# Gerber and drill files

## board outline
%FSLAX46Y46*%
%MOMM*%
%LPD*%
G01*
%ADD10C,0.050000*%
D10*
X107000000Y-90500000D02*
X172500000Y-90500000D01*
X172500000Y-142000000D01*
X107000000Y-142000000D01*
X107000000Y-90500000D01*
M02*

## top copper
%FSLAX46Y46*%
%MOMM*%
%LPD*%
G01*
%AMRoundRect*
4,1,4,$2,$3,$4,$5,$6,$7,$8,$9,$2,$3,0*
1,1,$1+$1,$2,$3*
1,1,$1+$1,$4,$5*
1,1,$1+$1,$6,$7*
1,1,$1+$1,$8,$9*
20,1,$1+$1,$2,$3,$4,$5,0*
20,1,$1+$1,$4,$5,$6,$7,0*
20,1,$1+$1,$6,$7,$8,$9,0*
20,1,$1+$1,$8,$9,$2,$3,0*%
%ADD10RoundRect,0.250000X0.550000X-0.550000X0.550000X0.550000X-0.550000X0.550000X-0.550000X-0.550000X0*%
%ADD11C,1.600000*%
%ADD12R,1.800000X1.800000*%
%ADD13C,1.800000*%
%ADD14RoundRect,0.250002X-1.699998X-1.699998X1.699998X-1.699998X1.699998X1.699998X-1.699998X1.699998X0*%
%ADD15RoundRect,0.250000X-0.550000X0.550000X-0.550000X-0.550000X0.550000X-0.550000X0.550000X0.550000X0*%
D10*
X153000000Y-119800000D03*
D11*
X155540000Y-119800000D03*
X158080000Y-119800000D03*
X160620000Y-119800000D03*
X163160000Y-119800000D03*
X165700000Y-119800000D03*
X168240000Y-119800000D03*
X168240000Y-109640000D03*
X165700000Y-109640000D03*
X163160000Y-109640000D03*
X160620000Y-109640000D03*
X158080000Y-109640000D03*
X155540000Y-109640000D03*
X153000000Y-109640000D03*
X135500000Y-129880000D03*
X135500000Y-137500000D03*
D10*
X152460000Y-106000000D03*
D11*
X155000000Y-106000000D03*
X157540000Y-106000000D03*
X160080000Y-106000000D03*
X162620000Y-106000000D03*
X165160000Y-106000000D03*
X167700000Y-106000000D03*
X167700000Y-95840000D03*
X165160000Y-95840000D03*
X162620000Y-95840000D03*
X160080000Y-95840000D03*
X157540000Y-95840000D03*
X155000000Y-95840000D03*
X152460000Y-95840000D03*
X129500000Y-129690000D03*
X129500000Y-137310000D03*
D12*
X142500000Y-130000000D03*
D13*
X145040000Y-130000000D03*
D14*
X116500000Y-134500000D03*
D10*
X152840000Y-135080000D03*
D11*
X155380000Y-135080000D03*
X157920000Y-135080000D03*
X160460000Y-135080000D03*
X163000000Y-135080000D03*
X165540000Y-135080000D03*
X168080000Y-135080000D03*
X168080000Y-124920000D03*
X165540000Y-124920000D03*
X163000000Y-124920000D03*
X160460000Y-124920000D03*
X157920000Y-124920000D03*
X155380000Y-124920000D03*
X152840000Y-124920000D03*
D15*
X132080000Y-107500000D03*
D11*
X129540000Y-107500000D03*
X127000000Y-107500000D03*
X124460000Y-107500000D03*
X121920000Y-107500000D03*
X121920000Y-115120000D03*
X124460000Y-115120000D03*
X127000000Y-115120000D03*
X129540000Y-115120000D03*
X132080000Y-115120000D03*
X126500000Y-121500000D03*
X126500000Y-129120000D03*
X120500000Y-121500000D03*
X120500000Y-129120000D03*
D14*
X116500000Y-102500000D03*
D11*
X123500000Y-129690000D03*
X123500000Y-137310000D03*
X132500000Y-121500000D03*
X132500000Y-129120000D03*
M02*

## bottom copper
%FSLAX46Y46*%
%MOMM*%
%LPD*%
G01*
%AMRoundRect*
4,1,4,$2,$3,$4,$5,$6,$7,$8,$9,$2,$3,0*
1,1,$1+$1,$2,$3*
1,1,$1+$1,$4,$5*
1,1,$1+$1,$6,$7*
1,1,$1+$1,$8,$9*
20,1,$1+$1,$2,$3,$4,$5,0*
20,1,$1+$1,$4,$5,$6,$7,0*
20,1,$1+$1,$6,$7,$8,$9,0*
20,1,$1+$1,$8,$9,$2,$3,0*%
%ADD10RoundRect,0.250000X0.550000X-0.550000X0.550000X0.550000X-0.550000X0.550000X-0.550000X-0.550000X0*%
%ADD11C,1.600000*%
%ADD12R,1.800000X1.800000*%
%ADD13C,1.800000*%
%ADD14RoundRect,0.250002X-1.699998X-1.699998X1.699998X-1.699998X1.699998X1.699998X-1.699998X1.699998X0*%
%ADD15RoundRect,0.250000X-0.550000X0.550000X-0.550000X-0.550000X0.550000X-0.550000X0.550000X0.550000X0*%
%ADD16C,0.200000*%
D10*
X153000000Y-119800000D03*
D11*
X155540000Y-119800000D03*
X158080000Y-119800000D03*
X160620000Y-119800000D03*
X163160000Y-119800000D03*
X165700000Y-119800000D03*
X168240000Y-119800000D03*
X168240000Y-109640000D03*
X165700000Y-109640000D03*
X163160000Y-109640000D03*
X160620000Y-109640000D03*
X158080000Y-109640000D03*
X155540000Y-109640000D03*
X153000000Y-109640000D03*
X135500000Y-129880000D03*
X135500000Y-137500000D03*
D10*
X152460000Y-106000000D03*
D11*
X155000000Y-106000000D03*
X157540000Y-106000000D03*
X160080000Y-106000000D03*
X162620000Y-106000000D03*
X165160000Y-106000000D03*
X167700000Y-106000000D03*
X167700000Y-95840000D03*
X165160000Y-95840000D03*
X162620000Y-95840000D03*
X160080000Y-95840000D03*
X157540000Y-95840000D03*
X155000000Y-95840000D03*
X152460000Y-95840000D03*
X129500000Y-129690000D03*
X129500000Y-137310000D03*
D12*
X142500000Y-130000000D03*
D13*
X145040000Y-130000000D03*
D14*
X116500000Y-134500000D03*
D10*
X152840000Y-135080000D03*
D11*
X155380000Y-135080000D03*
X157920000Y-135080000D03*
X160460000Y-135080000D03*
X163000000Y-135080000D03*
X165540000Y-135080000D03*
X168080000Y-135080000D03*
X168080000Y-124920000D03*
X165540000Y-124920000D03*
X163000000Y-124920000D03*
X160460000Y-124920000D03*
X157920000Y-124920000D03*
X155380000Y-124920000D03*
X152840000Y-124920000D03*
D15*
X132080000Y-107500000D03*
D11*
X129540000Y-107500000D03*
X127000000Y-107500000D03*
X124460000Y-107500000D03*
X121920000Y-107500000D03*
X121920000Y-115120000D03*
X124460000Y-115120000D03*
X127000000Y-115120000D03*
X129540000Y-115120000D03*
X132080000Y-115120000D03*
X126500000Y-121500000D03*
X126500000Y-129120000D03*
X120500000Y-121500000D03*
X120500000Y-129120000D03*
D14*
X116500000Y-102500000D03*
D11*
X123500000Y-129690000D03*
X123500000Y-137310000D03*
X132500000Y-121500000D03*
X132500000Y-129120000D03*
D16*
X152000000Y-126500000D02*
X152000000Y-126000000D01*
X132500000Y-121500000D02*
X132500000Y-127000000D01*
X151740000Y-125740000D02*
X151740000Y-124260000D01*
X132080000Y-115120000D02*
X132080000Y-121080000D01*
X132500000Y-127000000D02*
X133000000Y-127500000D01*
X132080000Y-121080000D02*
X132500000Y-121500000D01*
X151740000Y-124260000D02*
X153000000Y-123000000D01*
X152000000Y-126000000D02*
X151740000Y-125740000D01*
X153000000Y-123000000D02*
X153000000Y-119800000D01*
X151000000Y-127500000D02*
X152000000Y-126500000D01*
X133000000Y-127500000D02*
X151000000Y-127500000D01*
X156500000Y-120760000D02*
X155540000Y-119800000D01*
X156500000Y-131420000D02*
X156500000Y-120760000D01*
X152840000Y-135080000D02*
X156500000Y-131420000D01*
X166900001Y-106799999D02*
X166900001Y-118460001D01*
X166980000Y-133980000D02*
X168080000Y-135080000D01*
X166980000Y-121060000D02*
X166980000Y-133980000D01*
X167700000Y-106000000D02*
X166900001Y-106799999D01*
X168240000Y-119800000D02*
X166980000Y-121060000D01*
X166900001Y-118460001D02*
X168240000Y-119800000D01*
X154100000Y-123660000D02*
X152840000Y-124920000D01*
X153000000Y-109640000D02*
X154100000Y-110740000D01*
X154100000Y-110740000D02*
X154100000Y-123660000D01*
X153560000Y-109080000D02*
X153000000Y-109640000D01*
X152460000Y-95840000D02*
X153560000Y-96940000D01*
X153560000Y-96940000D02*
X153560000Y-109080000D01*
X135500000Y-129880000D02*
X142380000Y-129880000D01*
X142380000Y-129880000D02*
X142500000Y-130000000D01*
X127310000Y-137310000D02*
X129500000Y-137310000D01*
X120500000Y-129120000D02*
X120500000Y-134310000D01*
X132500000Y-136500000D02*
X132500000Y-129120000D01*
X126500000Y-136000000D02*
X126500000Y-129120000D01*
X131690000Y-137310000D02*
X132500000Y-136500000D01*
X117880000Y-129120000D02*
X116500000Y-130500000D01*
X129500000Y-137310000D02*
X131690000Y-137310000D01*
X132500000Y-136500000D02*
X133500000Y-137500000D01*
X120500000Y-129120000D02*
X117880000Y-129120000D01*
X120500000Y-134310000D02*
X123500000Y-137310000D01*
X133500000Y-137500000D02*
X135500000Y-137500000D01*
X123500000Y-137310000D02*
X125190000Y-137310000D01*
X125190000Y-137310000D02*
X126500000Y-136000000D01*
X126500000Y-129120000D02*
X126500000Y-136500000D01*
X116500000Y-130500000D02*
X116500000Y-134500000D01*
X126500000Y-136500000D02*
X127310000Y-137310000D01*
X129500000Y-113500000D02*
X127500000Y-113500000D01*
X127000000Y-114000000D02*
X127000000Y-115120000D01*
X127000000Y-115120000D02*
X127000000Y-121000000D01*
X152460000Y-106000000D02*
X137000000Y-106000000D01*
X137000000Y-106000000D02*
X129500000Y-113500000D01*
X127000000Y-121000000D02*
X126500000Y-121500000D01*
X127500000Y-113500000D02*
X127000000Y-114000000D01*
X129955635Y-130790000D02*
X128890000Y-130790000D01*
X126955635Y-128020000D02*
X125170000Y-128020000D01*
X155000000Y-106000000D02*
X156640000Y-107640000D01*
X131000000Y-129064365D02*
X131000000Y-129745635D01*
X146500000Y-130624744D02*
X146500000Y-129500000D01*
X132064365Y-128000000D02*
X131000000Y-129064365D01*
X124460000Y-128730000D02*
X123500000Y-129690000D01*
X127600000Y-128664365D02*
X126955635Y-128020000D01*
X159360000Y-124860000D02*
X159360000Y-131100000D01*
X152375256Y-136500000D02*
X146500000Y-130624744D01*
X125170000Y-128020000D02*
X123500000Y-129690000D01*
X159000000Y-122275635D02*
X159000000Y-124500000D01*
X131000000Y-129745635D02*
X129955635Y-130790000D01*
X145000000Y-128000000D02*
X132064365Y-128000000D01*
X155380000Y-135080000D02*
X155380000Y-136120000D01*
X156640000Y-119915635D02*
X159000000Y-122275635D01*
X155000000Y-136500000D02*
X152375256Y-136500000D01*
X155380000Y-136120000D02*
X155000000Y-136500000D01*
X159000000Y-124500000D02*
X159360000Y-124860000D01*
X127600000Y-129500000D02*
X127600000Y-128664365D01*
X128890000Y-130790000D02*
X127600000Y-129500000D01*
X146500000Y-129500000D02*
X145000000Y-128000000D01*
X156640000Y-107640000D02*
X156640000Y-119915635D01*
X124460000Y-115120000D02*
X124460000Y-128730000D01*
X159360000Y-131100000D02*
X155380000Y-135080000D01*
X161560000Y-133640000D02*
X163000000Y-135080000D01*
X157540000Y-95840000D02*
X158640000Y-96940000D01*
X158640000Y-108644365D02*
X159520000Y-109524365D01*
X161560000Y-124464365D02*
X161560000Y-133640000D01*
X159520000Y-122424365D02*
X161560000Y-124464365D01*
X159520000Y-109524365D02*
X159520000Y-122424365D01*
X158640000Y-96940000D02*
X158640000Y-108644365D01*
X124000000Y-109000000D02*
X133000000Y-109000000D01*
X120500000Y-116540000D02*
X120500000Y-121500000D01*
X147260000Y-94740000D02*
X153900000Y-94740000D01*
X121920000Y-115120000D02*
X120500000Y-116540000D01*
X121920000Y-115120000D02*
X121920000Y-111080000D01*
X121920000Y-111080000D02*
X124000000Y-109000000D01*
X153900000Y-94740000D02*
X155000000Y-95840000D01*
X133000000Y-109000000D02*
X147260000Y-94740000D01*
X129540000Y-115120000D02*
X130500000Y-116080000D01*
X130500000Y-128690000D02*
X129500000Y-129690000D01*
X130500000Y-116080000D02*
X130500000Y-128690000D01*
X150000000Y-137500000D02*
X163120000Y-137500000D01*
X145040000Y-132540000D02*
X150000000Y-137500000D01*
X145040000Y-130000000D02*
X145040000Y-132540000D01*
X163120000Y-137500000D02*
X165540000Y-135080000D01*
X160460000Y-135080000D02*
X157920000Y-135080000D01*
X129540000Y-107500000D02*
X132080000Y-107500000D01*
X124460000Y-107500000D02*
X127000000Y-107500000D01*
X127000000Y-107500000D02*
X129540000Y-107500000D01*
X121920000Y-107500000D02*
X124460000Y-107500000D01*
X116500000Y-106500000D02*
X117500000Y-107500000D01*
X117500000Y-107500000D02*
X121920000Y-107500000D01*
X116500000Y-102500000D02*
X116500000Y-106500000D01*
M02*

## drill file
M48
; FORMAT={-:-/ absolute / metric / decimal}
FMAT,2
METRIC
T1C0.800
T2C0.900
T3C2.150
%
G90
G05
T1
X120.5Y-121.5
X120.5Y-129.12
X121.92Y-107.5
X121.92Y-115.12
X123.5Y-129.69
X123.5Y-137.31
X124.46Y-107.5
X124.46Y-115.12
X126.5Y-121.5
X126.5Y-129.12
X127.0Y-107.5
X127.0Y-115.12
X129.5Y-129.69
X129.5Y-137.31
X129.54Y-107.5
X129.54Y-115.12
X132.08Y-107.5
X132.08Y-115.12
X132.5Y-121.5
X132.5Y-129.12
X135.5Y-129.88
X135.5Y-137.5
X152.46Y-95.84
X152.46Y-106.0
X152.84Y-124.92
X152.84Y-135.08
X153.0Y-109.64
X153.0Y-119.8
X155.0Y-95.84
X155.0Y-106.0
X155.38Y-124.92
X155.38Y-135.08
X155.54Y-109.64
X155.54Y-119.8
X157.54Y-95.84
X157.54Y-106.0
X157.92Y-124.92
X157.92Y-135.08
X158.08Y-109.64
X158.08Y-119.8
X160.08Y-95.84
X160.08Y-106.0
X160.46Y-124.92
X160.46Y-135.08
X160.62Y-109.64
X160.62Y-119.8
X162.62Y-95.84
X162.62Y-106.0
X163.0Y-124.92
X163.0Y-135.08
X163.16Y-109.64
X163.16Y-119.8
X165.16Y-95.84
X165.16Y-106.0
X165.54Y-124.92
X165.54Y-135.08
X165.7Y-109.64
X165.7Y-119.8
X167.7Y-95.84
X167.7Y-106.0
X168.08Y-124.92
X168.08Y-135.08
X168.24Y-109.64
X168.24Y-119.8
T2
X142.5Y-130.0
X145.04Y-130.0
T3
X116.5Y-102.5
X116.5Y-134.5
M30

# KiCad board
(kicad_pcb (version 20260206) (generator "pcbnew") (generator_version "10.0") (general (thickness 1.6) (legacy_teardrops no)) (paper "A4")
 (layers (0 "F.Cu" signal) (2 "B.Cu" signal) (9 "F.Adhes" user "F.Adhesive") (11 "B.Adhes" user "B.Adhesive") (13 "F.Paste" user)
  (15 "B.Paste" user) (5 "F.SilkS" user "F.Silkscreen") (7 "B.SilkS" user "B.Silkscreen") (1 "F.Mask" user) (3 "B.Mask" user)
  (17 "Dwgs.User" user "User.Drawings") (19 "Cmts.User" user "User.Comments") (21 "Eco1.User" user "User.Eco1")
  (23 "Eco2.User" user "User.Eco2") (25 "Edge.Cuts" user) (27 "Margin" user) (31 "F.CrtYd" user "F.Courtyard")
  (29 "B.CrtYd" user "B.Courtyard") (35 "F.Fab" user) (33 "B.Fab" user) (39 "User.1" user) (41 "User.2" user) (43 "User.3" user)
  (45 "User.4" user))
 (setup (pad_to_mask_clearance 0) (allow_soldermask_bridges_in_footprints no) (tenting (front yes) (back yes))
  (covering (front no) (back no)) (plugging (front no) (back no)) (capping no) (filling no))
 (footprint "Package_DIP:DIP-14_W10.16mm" (layer "F.Cu") (at 153 119.8 90)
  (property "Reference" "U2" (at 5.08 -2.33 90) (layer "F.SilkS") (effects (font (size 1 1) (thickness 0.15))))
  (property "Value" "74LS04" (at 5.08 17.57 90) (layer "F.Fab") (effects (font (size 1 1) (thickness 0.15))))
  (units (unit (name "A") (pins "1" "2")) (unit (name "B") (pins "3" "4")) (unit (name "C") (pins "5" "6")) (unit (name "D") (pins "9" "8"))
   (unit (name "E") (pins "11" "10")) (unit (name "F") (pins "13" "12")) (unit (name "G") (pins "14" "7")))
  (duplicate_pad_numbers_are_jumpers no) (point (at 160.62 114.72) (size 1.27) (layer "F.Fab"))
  (pad "1" thru_hole roundrect (at 0 0 90) (size 1.6 1.6) (drill 0.8) (layers "*.Cu" "*.Mask") (remove_unused_layers no)
   (roundrect_rratio 0.15625) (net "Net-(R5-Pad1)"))
  (pad "2" thru_hole circle (at 0 2.54 90) (size 1.6 1.6) (drill 0.8) (layers "*.Cu" "*.Mask") (remove_unused_layers no)
   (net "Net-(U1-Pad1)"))
  (pad "3" thru_hole circle (at 0 5.08 90) (size 1.6 1.6) (drill 0.8) (layers "*.Cu" "*.Mask") (remove_unused_layers no)
   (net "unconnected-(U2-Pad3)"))
  (pad "4" thru_hole circle (at 0 7.62 90) (size 1.6 1.6) (drill 0.8) (layers "*.Cu" "*.Mask") (remove_unused_layers no)
   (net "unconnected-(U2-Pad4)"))
  (pad "5" thru_hole circle (at 0 10.16 90) (size 1.6 1.6) (drill 0.8) (layers "*.Cu" "*.Mask") (remove_unused_layers no)
   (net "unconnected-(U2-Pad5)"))
  (pad "6" thru_hole circle (at 0 12.7 90) (size 1.6 1.6) (drill 0.8) (layers "*.Cu" "*.Mask") (remove_unused_layers no)
   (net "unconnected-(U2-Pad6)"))
  (pad "7" thru_hole circle (at 0 15.24 90) (size 1.6 1.6) (drill 0.8) (layers "*.Cu" "*.Mask") (remove_unused_layers no)
   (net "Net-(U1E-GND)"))
  (pad "8" thru_hole circle (at 10.16 15.24 90) (size 1.6 1.6) (drill 0.8) (layers "*.Cu" "*.Mask") (remove_unused_layers no)
   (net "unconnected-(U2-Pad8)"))
  (pad "9" thru_hole circle (at 10.16 12.7 90) (size 1.6 1.6) (drill 0.8) (layers "*.Cu" "*.Mask") (remove_unused_layers no)
   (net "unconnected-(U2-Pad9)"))
  (pad "10" thru_hole circle (at 10.16 10.16 90) (size 1.6 1.6) (drill 0.8) (layers "*.Cu" "*.Mask") (remove_unused_layers no)
   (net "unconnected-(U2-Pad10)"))
  (pad "11" thru_hole circle (at 10.16 7.62 90) (size 1.6 1.6) (drill 0.8) (layers "*.Cu" "*.Mask") (remove_unused_layers no)
   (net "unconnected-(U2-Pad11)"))
  (pad "12" thru_hole circle (at 10.16 5.08 90) (size 1.6 1.6) (drill 0.8) (layers "*.Cu" "*.Mask") (remove_unused_layers no)
   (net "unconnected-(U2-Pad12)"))
  (pad "13" thru_hole circle (at 10.16 2.54 90) (size 1.6 1.6) (drill 0.8) (layers "*.Cu" "*.Mask") (remove_unused_layers no)
   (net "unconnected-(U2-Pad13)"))
  (pad "14" thru_hole circle (at 10.16 0 90) (size 1.6 1.6) (drill 0.8) (layers "*.Cu" "*.Mask") (remove_unused_layers no)
   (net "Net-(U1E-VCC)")))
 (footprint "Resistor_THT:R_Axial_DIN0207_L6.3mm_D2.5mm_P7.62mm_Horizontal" (layer "F.Cu") (at 135.5 129.88 -90)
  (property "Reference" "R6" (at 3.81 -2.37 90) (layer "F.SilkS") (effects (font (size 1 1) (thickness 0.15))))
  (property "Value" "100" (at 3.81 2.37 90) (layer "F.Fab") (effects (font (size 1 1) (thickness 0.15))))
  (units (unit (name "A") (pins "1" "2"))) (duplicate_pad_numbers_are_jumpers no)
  (pad "1" thru_hole circle (at 0 0 270) (size 1.6 1.6) (drill 0.8) (layers "*.Cu" "*.Mask") (remove_unused_layers no) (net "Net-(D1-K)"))
  (pad "2" thru_hole circle (at 7.62 0 270) (size 1.6 1.6) (drill 0.8) (layers "*.Cu" "*.Mask") (remove_unused_layers no) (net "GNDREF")))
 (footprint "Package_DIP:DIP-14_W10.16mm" (layer "F.Cu") (at 152.46 106 90)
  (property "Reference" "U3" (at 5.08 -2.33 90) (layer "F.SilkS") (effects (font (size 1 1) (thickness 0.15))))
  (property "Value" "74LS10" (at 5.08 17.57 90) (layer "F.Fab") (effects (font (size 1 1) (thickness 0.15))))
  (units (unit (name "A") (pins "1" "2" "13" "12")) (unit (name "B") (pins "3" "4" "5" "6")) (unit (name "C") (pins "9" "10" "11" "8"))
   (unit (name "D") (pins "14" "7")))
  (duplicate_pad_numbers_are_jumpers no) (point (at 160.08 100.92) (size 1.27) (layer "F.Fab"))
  (pad "1" thru_hole roundrect (at 0 0 90) (size 1.6 1.6) (drill 0.8) (layers "*.Cu" "*.Mask") (remove_unused_layers no)
   (roundrect_rratio 0.15625) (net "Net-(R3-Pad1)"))
  (pad "2" thru_hole circle (at 0 2.54 90) (size 1.6 1.6) (drill 0.8) (layers "*.Cu" "*.Mask") (remove_unused_layers no)
   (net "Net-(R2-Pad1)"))
  (pad "3" thru_hole circle (at 0 5.08 90) (size 1.6 1.6) (drill 0.8) (layers "*.Cu" "*.Mask") (remove_unused_layers no)
   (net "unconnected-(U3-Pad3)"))
  (pad "4" thru_hole circle (at 0 7.62 90) (size 1.6 1.6) (drill 0.8) (layers "*.Cu" "*.Mask") (remove_unused_layers no)
   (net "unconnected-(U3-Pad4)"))
  (pad "5" thru_hole circle (at 0 10.16 90) (size 1.6 1.6) (drill 0.8) (layers "*.Cu" "*.Mask") (remove_unused_layers no)
   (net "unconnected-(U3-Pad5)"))
  (pad "6" thru_hole circle (at 0 12.7 90) (size 1.6 1.6) (drill 0.8) (layers "*.Cu" "*.Mask") (remove_unused_layers no)
   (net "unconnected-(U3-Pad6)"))
  (pad "7" thru_hole circle (at 0 15.24 90) (size 1.6 1.6) (drill 0.8) (layers "*.Cu" "*.Mask") (remove_unused_layers no)
   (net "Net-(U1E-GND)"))
  (pad "8" thru_hole circle (at 10.16 15.24 90) (size 1.6 1.6) (drill 0.8) (layers "*.Cu" "*.Mask") (remove_unused_layers no)
   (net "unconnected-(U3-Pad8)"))
  (pad "9" thru_hole circle (at 10.16 12.7 90) (size 1.6 1.6) (drill 0.8) (layers "*.Cu" "*.Mask") (remove_unused_layers no)
   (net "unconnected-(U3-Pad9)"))
  (pad "10" thru_hole circle (at 10.16 10.16 90) (size 1.6 1.6) (drill 0.8) (layers "*.Cu" "*.Mask") (remove_unused_layers no)
   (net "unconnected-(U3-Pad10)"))
  (pad "11" thru_hole circle (at 10.16 7.62 90) (size 1.6 1.6) (drill 0.8) (layers "*.Cu" "*.Mask") (remove_unused_layers no)
   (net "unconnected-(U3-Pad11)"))
  (pad "12" thru_hole circle (at 10.16 5.08 90) (size 1.6 1.6) (drill 0.8) (layers "*.Cu" "*.Mask") (remove_unused_layers no)
   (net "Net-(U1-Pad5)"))
  (pad "13" thru_hole circle (at 10.16 2.54 90) (size 1.6 1.6) (drill 0.8) (layers "*.Cu" "*.Mask") (remove_unused_layers no)
   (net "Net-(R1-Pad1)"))
  (pad "14" thru_hole circle (at 10.16 0 90) (size 1.6 1.6) (drill 0.8) (layers "*.Cu" "*.Mask") (remove_unused_layers no)
   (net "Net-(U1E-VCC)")))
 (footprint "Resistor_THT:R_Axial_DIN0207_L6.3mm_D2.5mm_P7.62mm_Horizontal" (layer "F.Cu") (at 129.5 129.69 -90)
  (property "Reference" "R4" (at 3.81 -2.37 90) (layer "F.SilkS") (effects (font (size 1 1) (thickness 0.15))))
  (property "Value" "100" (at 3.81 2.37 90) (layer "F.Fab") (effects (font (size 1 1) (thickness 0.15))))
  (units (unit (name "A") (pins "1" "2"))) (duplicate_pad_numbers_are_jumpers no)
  (pad "1" thru_hole circle (at 0 0 270) (size 1.6 1.6) (drill 0.8) (layers "*.Cu" "*.Mask") (remove_unused_layers no) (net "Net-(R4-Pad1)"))
  (pad "2" thru_hole circle (at 7.62 0 270) (size 1.6 1.6) (drill 0.8) (layers "*.Cu" "*.Mask") (remove_unused_layers no) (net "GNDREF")))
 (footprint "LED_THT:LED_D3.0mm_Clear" (layer "F.Cu") (at 142.5 130)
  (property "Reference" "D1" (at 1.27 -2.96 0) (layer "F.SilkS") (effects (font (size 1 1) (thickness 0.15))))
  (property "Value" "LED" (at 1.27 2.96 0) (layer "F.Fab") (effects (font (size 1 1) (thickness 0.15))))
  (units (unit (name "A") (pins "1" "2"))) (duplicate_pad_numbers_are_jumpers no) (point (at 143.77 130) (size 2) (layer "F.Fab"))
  (pad "1" thru_hole rect (at 0 0) (size 1.8 1.8) (drill 0.9) (layers "*.Cu" "*.Mask") (remove_unused_layers no) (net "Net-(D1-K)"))
  (pad "2" thru_hole circle (at 2.54 0) (size 1.8 1.8) (drill 0.9) (layers "*.Cu" "*.Mask") (remove_unused_layers no) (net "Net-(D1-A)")))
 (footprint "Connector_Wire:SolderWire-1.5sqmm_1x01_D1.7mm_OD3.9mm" (layer "F.Cu") (at 116.5 134.5)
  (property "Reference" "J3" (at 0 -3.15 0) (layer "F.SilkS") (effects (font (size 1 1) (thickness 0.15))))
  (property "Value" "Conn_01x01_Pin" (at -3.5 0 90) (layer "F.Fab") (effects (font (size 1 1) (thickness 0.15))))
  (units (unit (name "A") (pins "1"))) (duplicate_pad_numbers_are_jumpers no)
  (pad "1" thru_hole roundrect (at 0 0) (size 3.9 3.9) (drill 2.15) (layers "*.Cu" "*.Mask") (remove_unused_layers no)
   (roundrect_rratio 0.064103) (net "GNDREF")))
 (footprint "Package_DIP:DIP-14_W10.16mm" (layer "F.Cu") (at 152.84 135.08 90)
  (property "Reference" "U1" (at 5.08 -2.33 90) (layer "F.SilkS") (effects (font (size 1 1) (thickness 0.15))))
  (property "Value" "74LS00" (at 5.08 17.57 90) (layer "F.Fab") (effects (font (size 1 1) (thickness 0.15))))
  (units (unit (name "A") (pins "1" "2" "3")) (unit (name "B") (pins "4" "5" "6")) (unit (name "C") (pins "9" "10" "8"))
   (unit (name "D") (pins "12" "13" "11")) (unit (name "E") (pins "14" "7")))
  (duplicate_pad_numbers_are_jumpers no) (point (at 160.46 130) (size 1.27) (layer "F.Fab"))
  (pad "1" thru_hole roundrect (at 0 0 90) (size 1.6 1.6) (drill 0.8) (layers "*.Cu" "*.Mask") (remove_unused_layers no)
   (roundrect_rratio 0.15625) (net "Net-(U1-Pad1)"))
  (pad "2" thru_hole circle (at 0 2.54 90) (size 1.6 1.6) (drill 0.8) (layers "*.Cu" "*.Mask") (remove_unused_layers no)
   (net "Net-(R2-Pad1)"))
  (pad "3" thru_hole circle (at 0 5.08 90) (size 1.6 1.6) (drill 0.8) (layers "*.Cu" "*.Mask") (remove_unused_layers no)
   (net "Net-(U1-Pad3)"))
  (pad "4" thru_hole circle (at 0 7.62 90) (size 1.6 1.6) (drill 0.8) (layers "*.Cu" "*.Mask") (remove_unused_layers no)
   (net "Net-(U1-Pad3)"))
  (pad "5" thru_hole circle (at 0 10.16 90) (size 1.6 1.6) (drill 0.8) (layers "*.Cu" "*.Mask") (remove_unused_layers no)
   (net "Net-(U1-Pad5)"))
  (pad "6" thru_hole circle (at 0 12.7 90) (size 1.6 1.6) (drill 0.8) (layers "*.Cu" "*.Mask") (remove_unused_layers no) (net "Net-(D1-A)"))
  (pad "7" thru_hole circle (at 0 15.24 90) (size 1.6 1.6) (drill 0.8) (layers "*.Cu" "*.Mask") (remove_unused_layers no)
   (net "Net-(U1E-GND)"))
  (pad "8" thru_hole circle (at 10.16 15.24 90) (size 1.6 1.6) (drill 0.8) (layers "*.Cu" "*.Mask") (remove_unused_layers no)
   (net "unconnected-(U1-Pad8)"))
  (pad "9" thru_hole circle (at 10.16 12.7 90) (size 1.6 1.6) (drill 0.8) (layers "*.Cu" "*.Mask") (remove_unused_layers no)
   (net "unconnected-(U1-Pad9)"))
  (pad "10" thru_hole circle (at 10.16 10.16 90) (size 1.6 1.6) (drill 0.8) (layers "*.Cu" "*.Mask") (remove_unused_layers no)
   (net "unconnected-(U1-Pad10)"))
  (pad "11" thru_hole circle (at 10.16 7.62 90) (size 1.6 1.6) (drill 0.8) (layers "*.Cu" "*.Mask") (remove_unused_layers no)
   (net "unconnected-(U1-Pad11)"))
  (pad "12" thru_hole circle (at 10.16 5.08 90) (size 1.6 1.6) (drill 0.8) (layers "*.Cu" "*.Mask") (remove_unused_layers no)
   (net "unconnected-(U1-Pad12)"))
  (pad "13" thru_hole circle (at 10.16 2.54 90) (size 1.6 1.6) (drill 0.8) (layers "*.Cu" "*.Mask") (remove_unused_layers no)
   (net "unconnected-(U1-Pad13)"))
  (pad "14" thru_hole circle (at 10.16 0 90) (size 1.6 1.6) (drill 0.8) (layers "*.Cu" "*.Mask") (remove_unused_layers no)
   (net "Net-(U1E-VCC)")))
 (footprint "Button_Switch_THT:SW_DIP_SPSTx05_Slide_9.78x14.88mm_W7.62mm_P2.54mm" (layer "F.Cu") (at 132.08 107.5 -90)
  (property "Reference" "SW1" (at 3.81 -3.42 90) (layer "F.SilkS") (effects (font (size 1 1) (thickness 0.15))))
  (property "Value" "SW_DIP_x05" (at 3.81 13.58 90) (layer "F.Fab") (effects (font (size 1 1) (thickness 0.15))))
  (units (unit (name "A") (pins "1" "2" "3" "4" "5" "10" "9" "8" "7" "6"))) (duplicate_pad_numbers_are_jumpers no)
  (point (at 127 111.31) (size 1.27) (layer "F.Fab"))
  (pad "1" thru_hole roundrect (at 0 0 270) (size 1.6 1.6) (drill 0.8) (layers "*.Cu" "*.Mask") (remove_unused_layers no)
   (roundrect_rratio 0.15625) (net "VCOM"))
  (pad "2" thru_hole circle (at 0 2.54 270) (size 1.6 1.6) (drill 0.8) (layers "*.Cu" "*.Mask") (remove_unused_layers no) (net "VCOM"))
  (pad "3" thru_hole circle (at 0 5.08 270) (size 1.6 1.6) (drill 0.8) (layers "*.Cu" "*.Mask") (remove_unused_layers no) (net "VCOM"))
  (pad "4" thru_hole circle (at 0 7.62 270) (size 1.6 1.6) (drill 0.8) (layers "*.Cu" "*.Mask") (remove_unused_layers no) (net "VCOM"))
  (pad "5" thru_hole circle (at 0 10.16 270) (size 1.6 1.6) (drill 0.8) (layers "*.Cu" "*.Mask") (remove_unused_layers no) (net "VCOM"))
  (pad "6" thru_hole circle (at 7.62 10.16 270) (size 1.6 1.6) (drill 0.8) (layers "*.Cu" "*.Mask") (remove_unused_layers no)
   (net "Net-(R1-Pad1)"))
  (pad "7" thru_hole circle (at 7.62 7.62 270) (size 1.6 1.6) (drill 0.8) (layers "*.Cu" "*.Mask") (remove_unused_layers no)
   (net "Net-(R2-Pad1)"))
  (pad "8" thru_hole circle (at 7.62 5.08 270) (size 1.6 1.6) (drill 0.8) (layers "*.Cu" "*.Mask") (remove_unused_layers no)
   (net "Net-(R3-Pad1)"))
  (pad "9" thru_hole circle (at 7.62 2.54 270) (size 1.6 1.6) (drill 0.8) (layers "*.Cu" "*.Mask") (remove_unused_layers no)
   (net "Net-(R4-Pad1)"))
  (pad "10" thru_hole circle (at 7.62 0 270) (size 1.6 1.6) (drill 0.8) (layers "*.Cu" "*.Mask") (remove_unused_layers no)
   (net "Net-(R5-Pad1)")))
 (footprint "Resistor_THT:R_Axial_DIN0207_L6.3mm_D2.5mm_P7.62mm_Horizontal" (layer "F.Cu") (at 126.5 121.5 -90)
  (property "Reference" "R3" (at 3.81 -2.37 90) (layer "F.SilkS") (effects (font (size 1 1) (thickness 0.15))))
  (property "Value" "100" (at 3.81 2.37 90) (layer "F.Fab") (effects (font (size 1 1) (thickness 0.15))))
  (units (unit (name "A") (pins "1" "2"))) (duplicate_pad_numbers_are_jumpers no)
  (pad "1" thru_hole circle (at 0 0 270) (size 1.6 1.6) (drill 0.8) (layers "*.Cu" "*.Mask") (remove_unused_layers no) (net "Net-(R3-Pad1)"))
  (pad "2" thru_hole circle (at 7.62 0 270) (size 1.6 1.6) (drill 0.8) (layers "*.Cu" "*.Mask") (remove_unused_layers no) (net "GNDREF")))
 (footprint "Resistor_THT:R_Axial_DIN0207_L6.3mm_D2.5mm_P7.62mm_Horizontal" (layer "F.Cu") (at 120.5 121.5 -90)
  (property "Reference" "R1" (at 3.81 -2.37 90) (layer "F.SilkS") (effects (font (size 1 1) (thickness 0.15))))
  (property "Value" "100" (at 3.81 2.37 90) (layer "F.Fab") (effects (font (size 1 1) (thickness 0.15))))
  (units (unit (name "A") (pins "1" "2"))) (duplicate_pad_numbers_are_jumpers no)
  (pad "1" thru_hole circle (at 0 0 270) (size 1.6 1.6) (drill 0.8) (layers "*.Cu" "*.Mask") (remove_unused_layers no) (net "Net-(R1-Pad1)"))
  (pad "2" thru_hole circle (at 7.62 0 270) (size 1.6 1.6) (drill 0.8) (layers "*.Cu" "*.Mask") (remove_unused_layers no) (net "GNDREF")))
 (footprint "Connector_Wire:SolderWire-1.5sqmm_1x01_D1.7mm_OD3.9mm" (layer "F.Cu") (at 116.5 102.5)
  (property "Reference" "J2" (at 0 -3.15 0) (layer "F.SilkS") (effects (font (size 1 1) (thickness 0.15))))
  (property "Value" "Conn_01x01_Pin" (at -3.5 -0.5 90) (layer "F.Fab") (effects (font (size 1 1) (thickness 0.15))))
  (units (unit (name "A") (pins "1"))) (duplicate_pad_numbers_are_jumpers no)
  (pad "1" thru_hole roundrect (at 0 0) (size 3.9 3.9) (drill 2.15) (layers "*.Cu" "*.Mask") (remove_unused_layers no)
   (roundrect_rratio 0.064103) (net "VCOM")))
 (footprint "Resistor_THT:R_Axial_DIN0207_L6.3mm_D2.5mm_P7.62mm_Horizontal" (layer "F.Cu") (at 123.5 129.69 -90)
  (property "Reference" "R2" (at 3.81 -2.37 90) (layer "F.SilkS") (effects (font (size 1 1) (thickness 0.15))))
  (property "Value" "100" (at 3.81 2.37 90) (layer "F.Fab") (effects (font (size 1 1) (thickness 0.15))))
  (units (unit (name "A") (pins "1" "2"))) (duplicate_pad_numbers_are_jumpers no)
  (pad "1" thru_hole circle (at 0 0 270) (size 1.6 1.6) (drill 0.8) (layers "*.Cu" "*.Mask") (remove_unused_layers no) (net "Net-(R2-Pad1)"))
  (pad "2" thru_hole circle (at 7.62 0 270) (size 1.6 1.6) (drill 0.8) (layers "*.Cu" "*.Mask") (remove_unused_layers no) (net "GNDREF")))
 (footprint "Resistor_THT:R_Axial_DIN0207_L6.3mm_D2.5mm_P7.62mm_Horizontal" (layer "F.Cu") (at 132.5 121.5 -90)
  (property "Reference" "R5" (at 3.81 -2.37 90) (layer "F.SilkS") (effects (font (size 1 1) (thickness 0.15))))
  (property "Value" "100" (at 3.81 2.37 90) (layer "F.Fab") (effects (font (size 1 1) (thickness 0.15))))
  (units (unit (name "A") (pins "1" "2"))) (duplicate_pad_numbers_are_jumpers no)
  (pad "1" thru_hole circle (at 0 0 270) (size 1.6 1.6) (drill 0.8) (layers "*.Cu" "*.Mask") (remove_unused_layers no) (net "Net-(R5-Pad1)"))
  (pad "2" thru_hole circle (at 7.62 0 270) (size 1.6 1.6) (drill 0.8) (layers "*.Cu" "*.Mask") (remove_unused_layers no) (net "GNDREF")))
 (gr_rect (start 107 90.5) (end 172.5 142) (stroke (width 0.05) (type default)) (fill no) (layer "Edge.Cuts"))
 (segment (start 152 126.5) (end 152 126) (width 0.2) (layer "B.Cu") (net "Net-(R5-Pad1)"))
 (segment (start 132.5 121.5) (end 132.5 127) (width 0.2) (layer "B.Cu") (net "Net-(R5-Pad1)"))
 (segment (start 151.74 125.74) (end 151.74 124.26) (width 0.2) (layer "B.Cu") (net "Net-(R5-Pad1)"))
 (segment (start 132.08 115.12) (end 132.08 121.08) (width 0.2) (layer "B.Cu") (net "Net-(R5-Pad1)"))
 (segment (start 132.5 127) (end 133 127.5) (width 0.2) (layer "B.Cu") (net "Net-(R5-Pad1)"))
 (segment (start 132.08 121.08) (end 132.5 121.5) (width 0.2) (layer "B.Cu") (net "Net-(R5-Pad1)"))
 (segment (start 151.74 124.26) (end 153 123) (width 0.2) (layer "B.Cu") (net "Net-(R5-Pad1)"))
 (segment (start 152 126) (end 151.74 125.74) (width 0.2) (layer "B.Cu") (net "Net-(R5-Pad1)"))
 (segment (start 153 123) (end 153 119.8) (width 0.2) (layer "B.Cu") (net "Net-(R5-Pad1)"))
 (segment (start 151 127.5) (end 152 126.5) (width 0.2) (layer "B.Cu") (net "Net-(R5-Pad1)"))
 (segment (start 133 127.5) (end 151 127.5) (width 0.2) (layer "B.Cu") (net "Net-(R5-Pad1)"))
 (segment (start 156.5 120.76) (end 155.54 119.8) (width 0.2) (layer "B.Cu") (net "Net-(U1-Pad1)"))
 (segment (start 156.5 131.42) (end 156.5 120.76) (width 0.2) (layer "B.Cu") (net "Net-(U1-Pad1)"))
 (segment (start 152.84 135.08) (end 156.5 131.42) (width 0.2) (layer "B.Cu") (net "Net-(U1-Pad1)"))
 (segment (start 166.900001 106.799999) (end 166.900001 118.460001) (width 0.2) (layer "B.Cu") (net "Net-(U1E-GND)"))
 (segment (start 166.98 133.98) (end 168.08 135.08) (width 0.2) (layer "B.Cu") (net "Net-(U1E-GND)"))
 (segment (start 166.98 121.06) (end 166.98 133.98) (width 0.2) (layer "B.Cu") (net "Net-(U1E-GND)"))
 (segment (start 167.7 106) (end 166.900001 106.799999) (width 0.2) (layer "B.Cu") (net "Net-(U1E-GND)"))
 (segment (start 168.24 119.8) (end 166.98 121.06) (width 0.2) (layer "B.Cu") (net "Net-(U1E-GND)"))
 (segment (start 166.900001 118.460001) (end 168.24 119.8) (width 0.2) (layer "B.Cu") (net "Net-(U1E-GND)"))
 (segment (start 154.1 123.66) (end 152.84 124.92) (width 0.2) (layer "B.Cu") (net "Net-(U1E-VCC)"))
 (segment (start 153 109.64) (end 154.1 110.74) (width 0.2) (layer "B.Cu") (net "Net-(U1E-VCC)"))
 (segment (start 154.1 110.74) (end 154.1 123.66) (width 0.2) (layer "B.Cu") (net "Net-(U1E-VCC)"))
 (segment (start 153.56 109.08) (end 153 109.64) (width 0.2) (layer "B.Cu") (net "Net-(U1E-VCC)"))
 (segment (start 152.46 95.84) (end 153.56 96.94) (width 0.2) (layer "B.Cu") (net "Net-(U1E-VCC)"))
 (segment (start 153.56 96.94) (end 153.56 109.08) (width 0.2) (layer "B.Cu") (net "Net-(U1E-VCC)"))
 (segment (start 135.5 129.88) (end 142.38 129.88) (width 0.2) (layer "B.Cu") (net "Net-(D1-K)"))
 (segment (start 142.38 129.88) (end 142.5 130) (width 0.2) (layer "B.Cu") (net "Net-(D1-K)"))
 (segment (start 127.31 137.31) (end 129.5 137.31) (width 0.2) (layer "B.Cu") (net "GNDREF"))
 (segment (start 120.5 129.12) (end 120.5 134.31) (width 0.2) (layer "B.Cu") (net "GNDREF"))
 (segment (start 132.5 136.5) (end 132.5 129.12) (width 0.2) (layer "B.Cu") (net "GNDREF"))
 (segment (start 126.5 136) (end 126.5 129.12) (width 0.2) (layer "B.Cu") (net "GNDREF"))
 (segment (start 131.69 137.31) (end 132.5 136.5) (width 0.2) (layer "B.Cu") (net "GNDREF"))
 (segment (start 117.88 129.12) (end 116.5 130.5) (width 0.2) (layer "B.Cu") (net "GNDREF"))
 (segment (start 129.5 137.31) (end 131.69 137.31) (width 0.2) (layer "B.Cu") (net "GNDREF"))
 (segment (start 132.5 136.5) (end 133.5 137.5) (width 0.2) (layer "B.Cu") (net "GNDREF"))
 (segment (start 120.5 129.12) (end 117.88 129.12) (width 0.2) (layer "B.Cu") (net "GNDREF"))
 (segment (start 120.5 134.31) (end 123.5 137.31) (width 0.2) (layer "B.Cu") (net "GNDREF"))
 (segment (start 133.5 137.5) (end 135.5 137.5) (width 0.2) (layer "B.Cu") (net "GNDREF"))
 (segment (start 123.5 137.31) (end 125.19 137.31) (width 0.2) (layer "B.Cu") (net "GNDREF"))
 (segment (start 125.19 137.31) (end 126.5 136) (width 0.2) (layer "B.Cu") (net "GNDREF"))
 (segment (start 126.5 129.12) (end 126.5 136.5) (width 0.2) (layer "B.Cu") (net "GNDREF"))
 (segment (start 116.5 130.5) (end 116.5 134.5) (width 0.2) (layer "B.Cu") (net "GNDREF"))
 (segment (start 126.5 136.5) (end 127.31 137.31) (width 0.2) (layer "B.Cu") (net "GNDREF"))
 (segment (start 129.5 113.5) (end 127.5 113.5) (width 0.2) (layer "B.Cu") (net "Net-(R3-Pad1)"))
 (segment (start 127 114) (end 127 115.12) (width 0.2) (layer "B.Cu") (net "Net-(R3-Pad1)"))
 (segment (start 127 115.12) (end 127 121) (width 0.2) (layer "B.Cu") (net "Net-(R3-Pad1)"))
 (segment (start 152.46 106) (end 137 106) (width 0.2) (layer "B.Cu") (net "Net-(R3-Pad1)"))
 (segment (start 137 106) (end 129.5 113.5) (width 0.2) (layer "B.Cu") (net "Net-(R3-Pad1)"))
 (segment (start 127 121) (end 126.5 121.5) (width 0.2) (layer "B.Cu") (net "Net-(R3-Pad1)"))
 (segment (start 127.5 113.5) (end 127 114) (width 0.2) (layer "B.Cu") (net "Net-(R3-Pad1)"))
 (segment (start 129.955635 130.79) (end 128.89 130.79) (width 0.2) (layer "B.Cu") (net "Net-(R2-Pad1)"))
 (segment (start 126.955635 128.02) (end 125.17 128.02) (width 0.2) (layer "B.Cu") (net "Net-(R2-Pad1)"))
 (segment (start 155 106) (end 156.64 107.64) (width 0.2) (layer "B.Cu") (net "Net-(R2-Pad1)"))
 (segment (start 131 129.064365) (end 131 129.745635) (width 0.2) (layer "B.Cu") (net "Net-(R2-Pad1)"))
 (segment (start 146.5 130.624744) (end 146.5 129.5) (width 0.2) (layer "B.Cu") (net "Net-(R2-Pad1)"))
 (segment (start 132.064365 128) (end 131 129.064365) (width 0.2) (layer "B.Cu") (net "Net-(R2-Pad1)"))
 (segment (start 124.46 128.73) (end 123.5 129.69) (width 0.2) (layer "B.Cu") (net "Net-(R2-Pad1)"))
 (segment (start 127.6 128.664365) (end 126.955635 128.02) (width 0.2) (layer "B.Cu") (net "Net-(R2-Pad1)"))
 (segment (start 159.36 124.86) (end 159.36 131.1) (width 0.2) (layer "B.Cu") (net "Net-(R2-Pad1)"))
 (segment (start 152.375256 136.5) (end 146.5 130.624744) (width 0.2) (layer "B.Cu") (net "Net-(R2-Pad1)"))
 (segment (start 125.17 128.02) (end 123.5 129.69) (width 0.2) (layer "B.Cu") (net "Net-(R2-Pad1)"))
 (segment (start 159 122.275635) (end 159 124.5) (width 0.2) (layer "B.Cu") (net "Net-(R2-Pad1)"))
 (segment (start 131 129.745635) (end 129.955635 130.79) (width 0.2) (layer "B.Cu") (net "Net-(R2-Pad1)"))
 (segment (start 145 128) (end 132.064365 128) (width 0.2) (layer "B.Cu") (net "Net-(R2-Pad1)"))
 (segment (start 155.38 135.08) (end 155.38 136.12) (width 0.2) (layer "B.Cu") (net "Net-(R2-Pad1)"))
 (segment (start 156.64 119.915635) (end 159 122.275635) (width 0.2) (layer "B.Cu") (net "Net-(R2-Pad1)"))
 (segment (start 155 136.5) (end 152.375256 136.5) (width 0.2) (layer "B.Cu") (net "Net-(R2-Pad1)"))
 (segment (start 155.38 136.12) (end 155 136.5) (width 0.2) (layer "B.Cu") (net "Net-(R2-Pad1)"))
 (segment (start 159 124.5) (end 159.36 124.86) (width 0.2) (layer "B.Cu") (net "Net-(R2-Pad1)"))
 (segment (start 127.6 129.5) (end 127.6 128.664365) (width 0.2) (layer "B.Cu") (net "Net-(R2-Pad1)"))
 (segment (start 128.89 130.79) (end 127.6 129.5) (width 0.2) (layer "B.Cu") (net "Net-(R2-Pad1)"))
 (segment (start 146.5 129.5) (end 145 128) (width 0.2) (layer "B.Cu") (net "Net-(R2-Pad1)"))
 (segment (start 156.64 107.64) (end 156.64 119.915635) (width 0.2) (layer "B.Cu") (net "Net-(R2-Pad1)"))
 (segment (start 124.46 115.12) (end 124.46 128.73) (width 0.2) (layer "B.Cu") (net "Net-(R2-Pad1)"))
 (segment (start 159.36 131.1) (end 155.38 135.08) (width 0.2) (layer "B.Cu") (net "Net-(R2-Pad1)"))
 (segment (start 161.56 133.64) (end 163 135.08) (width 0.2) (layer "B.Cu") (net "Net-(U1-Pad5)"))
 (segment (start 157.54 95.84) (end 158.64 96.94) (width 0.2) (layer "B.Cu") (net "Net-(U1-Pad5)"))
 (segment (start 158.64 108.644365) (end 159.52 109.524365) (width 0.2) (layer "B.Cu") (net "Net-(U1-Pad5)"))
 (segment (start 161.56 124.464365) (end 161.56 133.64) (width 0.2) (layer "B.Cu") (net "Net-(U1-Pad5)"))
 (segment (start 159.52 122.424365) (end 161.56 124.464365) (width 0.2) (layer "B.Cu") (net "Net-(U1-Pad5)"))
 (segment (start 159.52 109.524365) (end 159.52 122.424365) (width 0.2) (layer "B.Cu") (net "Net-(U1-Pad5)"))
 (segment (start 158.64 96.94) (end 158.64 108.644365) (width 0.2) (layer "B.Cu") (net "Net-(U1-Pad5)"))
 (segment (start 124 109) (end 133 109) (width 0.2) (layer "B.Cu") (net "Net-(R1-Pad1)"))
 (segment (start 120.5 116.54) (end 120.5 121.5) (width 0.2) (layer "B.Cu") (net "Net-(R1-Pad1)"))
 (segment (start 147.26 94.74) (end 153.9 94.74) (width 0.2) (layer "B.Cu") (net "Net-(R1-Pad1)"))
 (segment (start 121.92 115.12) (end 120.5 116.54) (width 0.2) (layer "B.Cu") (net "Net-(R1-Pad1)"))
 (segment (start 121.92 115.12) (end 121.92 111.08) (width 0.2) (layer "B.Cu") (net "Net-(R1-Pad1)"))
 (segment (start 121.92 111.08) (end 124 109) (width 0.2) (layer "B.Cu") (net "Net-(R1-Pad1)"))
 (segment (start 153.9 94.74) (end 155 95.84) (width 0.2) (layer "B.Cu") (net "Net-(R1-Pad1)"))
 (segment (start 133 109) (end 147.26 94.74) (width 0.2) (layer "B.Cu") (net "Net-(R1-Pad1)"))
 (segment (start 129.54 115.12) (end 130.5 116.08) (width 0.2) (layer "B.Cu") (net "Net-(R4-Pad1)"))
 (segment (start 130.5 128.69) (end 129.5 129.69) (width 0.2) (layer "B.Cu") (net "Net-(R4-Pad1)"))
 (segment (start 130.5 116.08) (end 130.5 128.69) (width 0.2) (layer "B.Cu") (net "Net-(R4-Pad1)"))
 (segment (start 150 137.5) (end 163.12 137.5) (width 0.2) (layer "B.Cu") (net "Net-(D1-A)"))
 (segment (start 145.04 132.54) (end 150 137.5) (width 0.2) (layer "B.Cu") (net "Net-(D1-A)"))
 (segment (start 145.04 130) (end 145.04 132.54) (width 0.2) (layer "B.Cu") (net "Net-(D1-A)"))
 (segment (start 163.12 137.5) (end 165.54 135.08) (width 0.2) (layer "B.Cu") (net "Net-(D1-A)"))
 (segment (start 160.46 135.08) (end 157.92 135.08) (width 0.2) (layer "B.Cu") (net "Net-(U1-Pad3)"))
 (segment (start 129.54 107.5) (end 132.08 107.5) (width 0.2) (layer "B.Cu") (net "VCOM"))
 (segment (start 124.46 107.5) (end 127 107.5) (width 0.2) (layer "B.Cu") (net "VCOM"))
 (segment (start 127 107.5) (end 129.54 107.5) (width 0.2) (layer "B.Cu") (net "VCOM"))
 (segment (start 121.92 107.5) (end 124.46 107.5) (width 0.2) (layer "B.Cu") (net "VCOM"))
 (segment (start 116.5 106.5) (end 117.5 107.5) (width 0.2) (layer "B.Cu") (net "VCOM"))
 (segment (start 117.5 107.5) (end 121.92 107.5) (width 0.2) (layer "B.Cu") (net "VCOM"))
 (segment (start 116.5 102.5) (end 116.5 106.5) (width 0.2) (layer "B.Cu") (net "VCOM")))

